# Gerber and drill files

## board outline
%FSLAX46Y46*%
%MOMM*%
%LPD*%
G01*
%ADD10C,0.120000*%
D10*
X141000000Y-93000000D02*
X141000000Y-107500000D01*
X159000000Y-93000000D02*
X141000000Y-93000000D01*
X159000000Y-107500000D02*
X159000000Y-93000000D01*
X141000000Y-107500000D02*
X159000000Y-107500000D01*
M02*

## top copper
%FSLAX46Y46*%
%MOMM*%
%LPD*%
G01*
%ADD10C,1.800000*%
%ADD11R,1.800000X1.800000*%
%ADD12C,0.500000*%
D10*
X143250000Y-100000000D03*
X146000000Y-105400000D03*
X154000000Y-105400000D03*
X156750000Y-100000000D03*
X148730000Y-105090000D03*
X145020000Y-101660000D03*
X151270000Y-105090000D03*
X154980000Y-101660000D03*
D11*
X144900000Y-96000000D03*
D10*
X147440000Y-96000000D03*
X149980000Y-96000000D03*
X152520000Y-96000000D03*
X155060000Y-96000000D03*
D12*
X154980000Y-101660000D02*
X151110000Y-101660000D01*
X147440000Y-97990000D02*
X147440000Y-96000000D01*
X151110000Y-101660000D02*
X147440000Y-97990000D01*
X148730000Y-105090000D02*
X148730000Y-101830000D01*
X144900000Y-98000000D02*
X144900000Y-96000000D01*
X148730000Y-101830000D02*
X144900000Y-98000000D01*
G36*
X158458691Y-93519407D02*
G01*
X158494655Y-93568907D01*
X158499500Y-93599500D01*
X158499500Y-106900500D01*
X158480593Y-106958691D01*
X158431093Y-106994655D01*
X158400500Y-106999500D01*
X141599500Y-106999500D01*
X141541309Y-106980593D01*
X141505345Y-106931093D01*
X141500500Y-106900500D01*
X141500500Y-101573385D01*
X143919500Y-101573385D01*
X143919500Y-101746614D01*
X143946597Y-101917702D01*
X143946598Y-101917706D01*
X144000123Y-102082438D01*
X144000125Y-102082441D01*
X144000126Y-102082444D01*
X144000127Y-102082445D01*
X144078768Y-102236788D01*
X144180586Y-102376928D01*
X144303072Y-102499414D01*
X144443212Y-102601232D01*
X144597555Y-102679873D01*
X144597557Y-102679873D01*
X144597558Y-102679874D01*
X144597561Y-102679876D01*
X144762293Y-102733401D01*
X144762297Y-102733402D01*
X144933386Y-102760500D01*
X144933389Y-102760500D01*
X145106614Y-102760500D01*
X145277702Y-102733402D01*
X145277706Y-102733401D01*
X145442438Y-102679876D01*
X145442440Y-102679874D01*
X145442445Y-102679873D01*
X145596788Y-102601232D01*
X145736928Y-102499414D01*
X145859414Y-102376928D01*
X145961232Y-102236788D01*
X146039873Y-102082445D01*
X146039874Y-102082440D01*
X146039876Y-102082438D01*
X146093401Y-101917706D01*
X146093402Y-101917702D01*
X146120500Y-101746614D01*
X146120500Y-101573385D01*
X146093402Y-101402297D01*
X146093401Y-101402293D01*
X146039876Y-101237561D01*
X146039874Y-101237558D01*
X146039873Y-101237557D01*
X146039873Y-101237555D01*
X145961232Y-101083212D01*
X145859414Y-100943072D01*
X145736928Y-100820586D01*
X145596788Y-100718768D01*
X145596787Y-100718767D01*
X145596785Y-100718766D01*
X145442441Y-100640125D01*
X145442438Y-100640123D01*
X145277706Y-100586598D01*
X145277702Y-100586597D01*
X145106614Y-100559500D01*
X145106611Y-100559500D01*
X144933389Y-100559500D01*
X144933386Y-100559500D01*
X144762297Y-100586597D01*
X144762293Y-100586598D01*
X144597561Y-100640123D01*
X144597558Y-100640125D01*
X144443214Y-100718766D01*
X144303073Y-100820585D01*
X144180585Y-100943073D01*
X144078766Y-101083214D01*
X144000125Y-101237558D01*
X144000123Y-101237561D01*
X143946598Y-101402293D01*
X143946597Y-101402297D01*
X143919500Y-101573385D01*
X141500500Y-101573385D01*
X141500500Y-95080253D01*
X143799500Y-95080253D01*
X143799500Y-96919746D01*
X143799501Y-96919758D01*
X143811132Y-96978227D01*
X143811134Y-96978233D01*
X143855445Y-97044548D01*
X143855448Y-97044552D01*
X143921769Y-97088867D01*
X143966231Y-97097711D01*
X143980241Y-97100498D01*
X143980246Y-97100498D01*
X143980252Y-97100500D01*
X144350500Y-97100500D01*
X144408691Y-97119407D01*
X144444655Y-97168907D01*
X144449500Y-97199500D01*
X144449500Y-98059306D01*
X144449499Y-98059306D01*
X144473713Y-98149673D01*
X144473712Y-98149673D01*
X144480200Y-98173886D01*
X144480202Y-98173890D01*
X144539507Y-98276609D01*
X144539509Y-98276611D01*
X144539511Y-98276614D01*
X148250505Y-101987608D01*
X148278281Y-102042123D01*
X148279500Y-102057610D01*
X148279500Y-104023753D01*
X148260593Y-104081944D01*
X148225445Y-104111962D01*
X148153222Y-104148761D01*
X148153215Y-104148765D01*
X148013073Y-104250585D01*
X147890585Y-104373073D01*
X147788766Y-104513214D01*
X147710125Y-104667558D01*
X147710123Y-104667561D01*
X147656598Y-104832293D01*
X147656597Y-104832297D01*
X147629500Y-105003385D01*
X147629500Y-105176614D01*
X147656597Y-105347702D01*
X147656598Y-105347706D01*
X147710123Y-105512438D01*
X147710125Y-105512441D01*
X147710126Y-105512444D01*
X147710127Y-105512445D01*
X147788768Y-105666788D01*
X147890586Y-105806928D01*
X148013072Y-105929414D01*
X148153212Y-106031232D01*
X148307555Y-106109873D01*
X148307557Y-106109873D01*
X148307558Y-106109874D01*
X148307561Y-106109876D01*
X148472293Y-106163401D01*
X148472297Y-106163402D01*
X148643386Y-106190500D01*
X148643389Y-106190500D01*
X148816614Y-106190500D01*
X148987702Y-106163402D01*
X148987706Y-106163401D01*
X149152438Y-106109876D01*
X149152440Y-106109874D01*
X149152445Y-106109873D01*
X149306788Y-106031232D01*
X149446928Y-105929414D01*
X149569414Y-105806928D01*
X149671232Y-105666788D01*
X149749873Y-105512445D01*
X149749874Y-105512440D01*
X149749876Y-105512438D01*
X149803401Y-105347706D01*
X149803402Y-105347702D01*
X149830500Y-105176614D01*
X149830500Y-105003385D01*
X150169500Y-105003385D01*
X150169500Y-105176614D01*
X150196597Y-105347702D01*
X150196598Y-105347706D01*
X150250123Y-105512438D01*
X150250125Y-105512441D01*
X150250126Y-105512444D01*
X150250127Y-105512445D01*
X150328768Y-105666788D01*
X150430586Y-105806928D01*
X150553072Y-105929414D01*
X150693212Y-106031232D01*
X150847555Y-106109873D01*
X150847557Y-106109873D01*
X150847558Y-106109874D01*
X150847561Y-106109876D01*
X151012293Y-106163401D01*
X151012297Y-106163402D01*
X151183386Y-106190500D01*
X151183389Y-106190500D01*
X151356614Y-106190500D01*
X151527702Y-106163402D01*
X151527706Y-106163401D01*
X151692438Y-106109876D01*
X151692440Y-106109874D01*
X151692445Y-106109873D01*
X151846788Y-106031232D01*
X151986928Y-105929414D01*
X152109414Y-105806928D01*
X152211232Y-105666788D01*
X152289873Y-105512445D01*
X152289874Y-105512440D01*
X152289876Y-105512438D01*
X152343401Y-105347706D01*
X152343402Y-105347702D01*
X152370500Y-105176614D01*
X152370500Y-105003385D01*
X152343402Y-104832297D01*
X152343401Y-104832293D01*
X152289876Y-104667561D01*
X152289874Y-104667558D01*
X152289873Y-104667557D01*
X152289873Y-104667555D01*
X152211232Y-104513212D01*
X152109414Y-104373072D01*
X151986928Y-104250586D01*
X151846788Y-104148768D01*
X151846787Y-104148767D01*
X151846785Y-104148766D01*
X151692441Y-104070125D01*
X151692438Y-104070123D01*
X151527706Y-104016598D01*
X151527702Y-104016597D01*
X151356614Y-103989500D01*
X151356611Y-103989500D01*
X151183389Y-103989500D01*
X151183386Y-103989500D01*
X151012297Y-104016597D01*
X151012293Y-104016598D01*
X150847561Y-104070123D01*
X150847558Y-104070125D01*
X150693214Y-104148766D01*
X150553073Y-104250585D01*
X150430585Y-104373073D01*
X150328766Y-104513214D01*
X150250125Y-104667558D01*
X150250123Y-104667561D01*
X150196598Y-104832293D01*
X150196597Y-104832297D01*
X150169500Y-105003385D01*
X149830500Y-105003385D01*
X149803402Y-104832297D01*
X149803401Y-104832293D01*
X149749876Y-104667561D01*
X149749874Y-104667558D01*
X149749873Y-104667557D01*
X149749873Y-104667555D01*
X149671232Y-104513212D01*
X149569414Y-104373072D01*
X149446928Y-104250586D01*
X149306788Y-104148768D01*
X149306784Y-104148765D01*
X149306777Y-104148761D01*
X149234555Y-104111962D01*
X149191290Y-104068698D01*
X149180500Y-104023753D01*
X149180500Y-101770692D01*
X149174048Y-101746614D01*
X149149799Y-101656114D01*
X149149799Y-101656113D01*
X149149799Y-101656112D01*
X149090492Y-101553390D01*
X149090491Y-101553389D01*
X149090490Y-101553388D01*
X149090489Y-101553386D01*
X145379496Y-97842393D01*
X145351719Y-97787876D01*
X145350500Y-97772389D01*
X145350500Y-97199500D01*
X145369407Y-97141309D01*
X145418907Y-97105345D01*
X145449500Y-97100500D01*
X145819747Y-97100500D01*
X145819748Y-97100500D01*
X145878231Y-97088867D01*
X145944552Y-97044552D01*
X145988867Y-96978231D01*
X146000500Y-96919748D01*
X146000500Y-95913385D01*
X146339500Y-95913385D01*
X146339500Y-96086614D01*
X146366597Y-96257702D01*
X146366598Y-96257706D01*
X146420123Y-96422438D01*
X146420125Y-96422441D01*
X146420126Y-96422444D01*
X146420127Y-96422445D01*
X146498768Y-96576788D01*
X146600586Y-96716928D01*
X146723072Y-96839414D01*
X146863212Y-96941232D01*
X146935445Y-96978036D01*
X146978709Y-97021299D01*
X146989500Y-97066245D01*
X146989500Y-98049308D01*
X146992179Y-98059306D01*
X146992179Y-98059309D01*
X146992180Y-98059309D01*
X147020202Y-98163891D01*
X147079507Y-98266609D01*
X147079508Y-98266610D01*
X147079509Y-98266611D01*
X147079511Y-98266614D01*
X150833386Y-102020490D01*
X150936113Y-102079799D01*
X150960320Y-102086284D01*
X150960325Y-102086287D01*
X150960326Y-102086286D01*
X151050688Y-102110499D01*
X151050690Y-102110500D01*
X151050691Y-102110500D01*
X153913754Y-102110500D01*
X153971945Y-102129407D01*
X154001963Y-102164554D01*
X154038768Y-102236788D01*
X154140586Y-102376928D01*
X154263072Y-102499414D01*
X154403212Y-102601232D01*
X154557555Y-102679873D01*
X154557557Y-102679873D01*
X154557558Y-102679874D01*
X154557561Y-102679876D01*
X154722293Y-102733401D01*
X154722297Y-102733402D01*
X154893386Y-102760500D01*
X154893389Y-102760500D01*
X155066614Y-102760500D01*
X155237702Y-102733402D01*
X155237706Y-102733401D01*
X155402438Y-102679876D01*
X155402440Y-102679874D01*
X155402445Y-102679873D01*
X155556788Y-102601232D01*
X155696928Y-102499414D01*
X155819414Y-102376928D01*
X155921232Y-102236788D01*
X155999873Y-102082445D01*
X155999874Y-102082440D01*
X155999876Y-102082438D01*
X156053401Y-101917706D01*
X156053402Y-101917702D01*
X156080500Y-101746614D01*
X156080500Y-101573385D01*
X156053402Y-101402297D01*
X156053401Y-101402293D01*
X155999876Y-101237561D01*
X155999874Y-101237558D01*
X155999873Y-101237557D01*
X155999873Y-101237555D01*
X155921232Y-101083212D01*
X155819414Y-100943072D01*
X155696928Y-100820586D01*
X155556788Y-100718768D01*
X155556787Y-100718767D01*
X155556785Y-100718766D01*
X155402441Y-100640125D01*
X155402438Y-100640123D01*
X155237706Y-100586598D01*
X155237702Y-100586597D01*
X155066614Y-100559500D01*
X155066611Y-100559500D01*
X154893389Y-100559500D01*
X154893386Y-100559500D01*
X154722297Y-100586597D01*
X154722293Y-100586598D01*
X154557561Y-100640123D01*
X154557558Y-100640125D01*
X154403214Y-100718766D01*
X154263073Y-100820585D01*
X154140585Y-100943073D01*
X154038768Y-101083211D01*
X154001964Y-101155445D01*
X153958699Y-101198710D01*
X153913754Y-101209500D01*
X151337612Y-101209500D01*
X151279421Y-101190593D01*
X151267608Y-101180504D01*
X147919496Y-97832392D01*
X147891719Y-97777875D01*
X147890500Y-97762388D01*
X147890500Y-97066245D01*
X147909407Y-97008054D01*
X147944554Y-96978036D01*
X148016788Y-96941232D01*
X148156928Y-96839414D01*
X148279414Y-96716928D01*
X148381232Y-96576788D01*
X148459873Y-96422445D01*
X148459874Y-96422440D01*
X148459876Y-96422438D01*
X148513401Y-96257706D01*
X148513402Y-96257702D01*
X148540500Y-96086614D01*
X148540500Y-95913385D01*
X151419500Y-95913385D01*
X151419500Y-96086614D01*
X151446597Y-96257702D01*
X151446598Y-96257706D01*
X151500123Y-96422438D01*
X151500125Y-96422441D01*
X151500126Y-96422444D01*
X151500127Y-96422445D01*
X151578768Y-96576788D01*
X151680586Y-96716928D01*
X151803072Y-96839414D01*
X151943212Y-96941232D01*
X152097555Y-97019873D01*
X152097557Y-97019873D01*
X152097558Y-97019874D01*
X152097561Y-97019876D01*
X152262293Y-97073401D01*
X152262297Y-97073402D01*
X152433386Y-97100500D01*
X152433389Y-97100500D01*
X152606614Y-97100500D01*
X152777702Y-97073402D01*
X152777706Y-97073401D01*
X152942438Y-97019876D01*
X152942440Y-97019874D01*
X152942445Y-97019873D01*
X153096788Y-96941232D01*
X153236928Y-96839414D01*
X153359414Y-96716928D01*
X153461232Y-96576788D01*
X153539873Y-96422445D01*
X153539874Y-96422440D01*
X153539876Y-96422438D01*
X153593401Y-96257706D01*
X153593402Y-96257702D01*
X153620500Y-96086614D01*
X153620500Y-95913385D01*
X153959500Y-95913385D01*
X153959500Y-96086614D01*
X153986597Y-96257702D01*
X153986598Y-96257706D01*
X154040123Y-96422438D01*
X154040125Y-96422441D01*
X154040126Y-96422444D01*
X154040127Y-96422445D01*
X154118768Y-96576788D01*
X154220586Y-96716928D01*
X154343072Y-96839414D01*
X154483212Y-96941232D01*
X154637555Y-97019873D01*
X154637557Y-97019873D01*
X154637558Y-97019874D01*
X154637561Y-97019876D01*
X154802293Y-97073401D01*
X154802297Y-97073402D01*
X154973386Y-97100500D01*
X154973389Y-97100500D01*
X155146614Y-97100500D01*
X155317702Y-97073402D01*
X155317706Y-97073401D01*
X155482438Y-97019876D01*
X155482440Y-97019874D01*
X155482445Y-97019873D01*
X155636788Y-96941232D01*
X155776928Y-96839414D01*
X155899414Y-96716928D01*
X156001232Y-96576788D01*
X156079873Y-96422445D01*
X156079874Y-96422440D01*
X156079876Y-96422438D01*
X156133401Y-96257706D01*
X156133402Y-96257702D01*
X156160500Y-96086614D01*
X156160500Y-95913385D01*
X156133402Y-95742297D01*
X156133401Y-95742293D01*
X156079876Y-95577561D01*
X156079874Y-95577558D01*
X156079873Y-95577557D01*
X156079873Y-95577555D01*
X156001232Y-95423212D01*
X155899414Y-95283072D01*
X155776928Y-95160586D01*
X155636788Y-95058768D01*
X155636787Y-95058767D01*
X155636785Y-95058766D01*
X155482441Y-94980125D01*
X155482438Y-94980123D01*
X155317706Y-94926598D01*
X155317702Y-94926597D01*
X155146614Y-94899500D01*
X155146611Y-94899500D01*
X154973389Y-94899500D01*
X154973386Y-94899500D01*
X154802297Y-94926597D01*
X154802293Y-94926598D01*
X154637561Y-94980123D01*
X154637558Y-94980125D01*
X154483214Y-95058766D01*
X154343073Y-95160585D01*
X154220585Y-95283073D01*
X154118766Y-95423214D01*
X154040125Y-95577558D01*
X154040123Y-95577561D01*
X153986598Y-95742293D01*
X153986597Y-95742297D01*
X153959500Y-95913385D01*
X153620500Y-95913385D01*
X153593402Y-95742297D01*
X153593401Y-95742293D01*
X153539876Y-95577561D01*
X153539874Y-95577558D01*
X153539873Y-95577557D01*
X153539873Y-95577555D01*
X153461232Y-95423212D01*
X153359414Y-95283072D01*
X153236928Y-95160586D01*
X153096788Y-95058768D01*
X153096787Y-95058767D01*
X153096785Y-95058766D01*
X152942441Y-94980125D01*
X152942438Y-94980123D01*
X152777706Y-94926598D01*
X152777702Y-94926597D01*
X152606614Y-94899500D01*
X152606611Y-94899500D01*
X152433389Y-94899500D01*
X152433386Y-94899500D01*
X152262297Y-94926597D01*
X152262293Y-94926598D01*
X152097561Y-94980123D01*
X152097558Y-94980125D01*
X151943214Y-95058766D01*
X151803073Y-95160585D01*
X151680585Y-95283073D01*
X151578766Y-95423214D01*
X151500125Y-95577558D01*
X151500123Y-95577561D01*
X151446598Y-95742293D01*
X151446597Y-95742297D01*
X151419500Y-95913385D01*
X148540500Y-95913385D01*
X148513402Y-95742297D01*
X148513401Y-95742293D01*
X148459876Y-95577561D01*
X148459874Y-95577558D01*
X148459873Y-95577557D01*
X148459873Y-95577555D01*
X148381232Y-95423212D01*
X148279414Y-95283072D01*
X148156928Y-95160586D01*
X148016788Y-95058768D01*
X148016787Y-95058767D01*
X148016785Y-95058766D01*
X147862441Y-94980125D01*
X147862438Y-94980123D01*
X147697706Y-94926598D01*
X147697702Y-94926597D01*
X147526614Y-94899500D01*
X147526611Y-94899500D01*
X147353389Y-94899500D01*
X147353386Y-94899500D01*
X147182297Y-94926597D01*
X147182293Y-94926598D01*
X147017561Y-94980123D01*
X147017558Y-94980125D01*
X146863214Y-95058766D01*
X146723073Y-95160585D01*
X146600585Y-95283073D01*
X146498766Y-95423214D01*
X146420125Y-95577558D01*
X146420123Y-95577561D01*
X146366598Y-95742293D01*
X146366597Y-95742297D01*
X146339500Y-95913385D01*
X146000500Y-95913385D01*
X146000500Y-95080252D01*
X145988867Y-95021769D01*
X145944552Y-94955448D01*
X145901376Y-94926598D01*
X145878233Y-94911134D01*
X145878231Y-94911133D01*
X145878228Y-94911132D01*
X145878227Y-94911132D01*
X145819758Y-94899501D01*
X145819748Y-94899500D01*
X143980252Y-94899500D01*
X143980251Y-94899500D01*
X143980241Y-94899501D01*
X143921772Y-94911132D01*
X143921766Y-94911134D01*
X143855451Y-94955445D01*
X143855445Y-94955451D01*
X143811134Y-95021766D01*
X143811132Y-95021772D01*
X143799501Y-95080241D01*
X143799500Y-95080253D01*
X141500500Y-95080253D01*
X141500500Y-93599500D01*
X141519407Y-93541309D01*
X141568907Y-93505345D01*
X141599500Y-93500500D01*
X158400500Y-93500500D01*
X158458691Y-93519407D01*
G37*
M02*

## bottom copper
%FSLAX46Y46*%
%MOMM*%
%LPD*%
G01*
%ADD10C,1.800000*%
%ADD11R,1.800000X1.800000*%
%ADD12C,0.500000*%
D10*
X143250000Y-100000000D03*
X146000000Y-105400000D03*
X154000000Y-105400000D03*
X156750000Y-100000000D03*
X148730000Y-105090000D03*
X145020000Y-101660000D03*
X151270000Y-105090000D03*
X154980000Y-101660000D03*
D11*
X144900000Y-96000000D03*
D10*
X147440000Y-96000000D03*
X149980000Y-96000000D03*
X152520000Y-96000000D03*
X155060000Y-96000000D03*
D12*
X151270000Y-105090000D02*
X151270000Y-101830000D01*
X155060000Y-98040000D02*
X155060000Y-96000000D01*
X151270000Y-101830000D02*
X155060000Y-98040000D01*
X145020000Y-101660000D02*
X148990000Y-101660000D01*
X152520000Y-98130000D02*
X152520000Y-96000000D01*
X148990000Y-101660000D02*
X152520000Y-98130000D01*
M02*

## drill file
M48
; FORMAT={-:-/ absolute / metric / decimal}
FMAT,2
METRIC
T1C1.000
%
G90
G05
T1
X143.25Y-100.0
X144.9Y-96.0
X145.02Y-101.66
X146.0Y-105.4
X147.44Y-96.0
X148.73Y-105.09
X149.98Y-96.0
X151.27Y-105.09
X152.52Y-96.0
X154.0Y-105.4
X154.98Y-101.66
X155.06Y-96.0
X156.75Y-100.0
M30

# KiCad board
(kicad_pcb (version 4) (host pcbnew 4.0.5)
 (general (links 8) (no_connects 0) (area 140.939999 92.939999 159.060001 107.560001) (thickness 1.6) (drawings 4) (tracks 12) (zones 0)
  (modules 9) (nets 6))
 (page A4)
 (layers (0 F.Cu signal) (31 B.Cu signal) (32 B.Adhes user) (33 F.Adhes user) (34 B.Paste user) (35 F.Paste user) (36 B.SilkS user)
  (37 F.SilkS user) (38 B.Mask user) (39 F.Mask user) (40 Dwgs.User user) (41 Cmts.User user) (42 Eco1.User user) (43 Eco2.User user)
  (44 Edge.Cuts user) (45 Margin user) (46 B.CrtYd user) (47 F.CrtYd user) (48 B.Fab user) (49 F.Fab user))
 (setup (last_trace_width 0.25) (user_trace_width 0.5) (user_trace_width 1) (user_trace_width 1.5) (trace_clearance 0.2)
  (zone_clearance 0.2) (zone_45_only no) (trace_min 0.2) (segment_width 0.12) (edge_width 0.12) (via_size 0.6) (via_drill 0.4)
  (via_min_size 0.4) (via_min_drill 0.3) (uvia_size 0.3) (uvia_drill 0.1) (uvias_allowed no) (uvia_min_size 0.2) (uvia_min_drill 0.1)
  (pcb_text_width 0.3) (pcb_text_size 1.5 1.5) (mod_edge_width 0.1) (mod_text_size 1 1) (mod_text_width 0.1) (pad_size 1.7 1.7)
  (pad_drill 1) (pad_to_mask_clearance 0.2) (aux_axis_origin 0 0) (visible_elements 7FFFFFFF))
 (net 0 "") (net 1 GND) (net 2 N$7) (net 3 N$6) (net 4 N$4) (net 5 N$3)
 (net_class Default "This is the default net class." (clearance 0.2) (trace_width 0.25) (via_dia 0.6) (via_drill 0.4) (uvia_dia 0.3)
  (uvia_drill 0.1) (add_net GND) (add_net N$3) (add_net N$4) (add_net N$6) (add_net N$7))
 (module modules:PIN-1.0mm (layer F.Cu) (at 143.25 100)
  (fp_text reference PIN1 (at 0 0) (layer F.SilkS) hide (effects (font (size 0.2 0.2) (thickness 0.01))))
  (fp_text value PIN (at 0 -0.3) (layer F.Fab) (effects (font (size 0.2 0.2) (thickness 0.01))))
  (pad 1 thru_hole circle (at 0 0) (size 1.8 1.8) (drill 1) (layers *.Cu *.Mask) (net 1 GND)))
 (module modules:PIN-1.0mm (layer F.Cu) (at 146 105.4)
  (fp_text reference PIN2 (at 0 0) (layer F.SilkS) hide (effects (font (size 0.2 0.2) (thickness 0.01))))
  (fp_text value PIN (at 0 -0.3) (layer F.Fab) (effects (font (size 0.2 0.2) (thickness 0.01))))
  (pad 1 thru_hole circle (at 0 0) (size 1.8 1.8) (drill 1) (layers *.Cu *.Mask) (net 1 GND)))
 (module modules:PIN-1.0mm (layer F.Cu) (at 154 105.4)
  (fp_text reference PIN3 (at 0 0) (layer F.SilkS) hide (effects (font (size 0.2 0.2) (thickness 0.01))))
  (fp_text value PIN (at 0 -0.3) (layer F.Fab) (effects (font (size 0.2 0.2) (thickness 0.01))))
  (pad 1 thru_hole circle (at 0 0) (size 1.8 1.8) (drill 1) (layers *.Cu *.Mask) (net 1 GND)))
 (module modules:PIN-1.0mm (layer F.Cu) (at 156.75 100)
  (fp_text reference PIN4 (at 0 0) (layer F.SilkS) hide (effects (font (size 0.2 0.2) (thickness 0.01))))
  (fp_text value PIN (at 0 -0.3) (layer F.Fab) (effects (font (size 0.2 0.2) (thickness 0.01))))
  (pad 1 thru_hole circle (at 0 0) (size 1.8 1.8) (drill 1) (layers *.Cu *.Mask) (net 1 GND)))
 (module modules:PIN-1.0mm (layer F.Cu) (at 148.73 105.09)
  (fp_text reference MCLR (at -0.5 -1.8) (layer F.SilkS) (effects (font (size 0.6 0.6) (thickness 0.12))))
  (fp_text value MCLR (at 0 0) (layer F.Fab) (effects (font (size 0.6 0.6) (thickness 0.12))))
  (pad 1 thru_hole circle (at 0 0) (size 1.8 1.8) (drill 1) (layers *.Cu *.Mask) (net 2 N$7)))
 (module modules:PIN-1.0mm (layer F.Cu) (at 145.02 101.66)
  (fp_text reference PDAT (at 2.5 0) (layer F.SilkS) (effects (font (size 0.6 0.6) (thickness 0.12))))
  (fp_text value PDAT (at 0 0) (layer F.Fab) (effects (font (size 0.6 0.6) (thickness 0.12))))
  (pad 1 thru_hole circle (at 0 0) (size 1.8 1.8) (drill 1) (layers *.Cu *.Mask) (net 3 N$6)))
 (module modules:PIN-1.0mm (layer F.Cu) (at 151.27 105.09)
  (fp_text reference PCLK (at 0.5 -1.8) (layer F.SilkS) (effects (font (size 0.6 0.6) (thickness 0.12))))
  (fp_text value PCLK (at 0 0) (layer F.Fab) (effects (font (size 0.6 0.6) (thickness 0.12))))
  (pad 1 thru_hole circle (at 0 0) (size 1.8 1.8) (drill 1) (layers *.Cu *.Mask) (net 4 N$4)))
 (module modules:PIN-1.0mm (layer F.Cu) (at 154.98 101.66)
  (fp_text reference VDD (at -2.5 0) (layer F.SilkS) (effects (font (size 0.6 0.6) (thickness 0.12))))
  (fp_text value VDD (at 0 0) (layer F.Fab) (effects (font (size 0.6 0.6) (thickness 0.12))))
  (pad 1 thru_hole circle (at 0 0) (size 1.8 1.8) (drill 1) (layers *.Cu *.Mask) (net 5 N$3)))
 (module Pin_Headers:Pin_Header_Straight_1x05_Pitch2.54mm (layer F.Cu) (at 144.9 96 90)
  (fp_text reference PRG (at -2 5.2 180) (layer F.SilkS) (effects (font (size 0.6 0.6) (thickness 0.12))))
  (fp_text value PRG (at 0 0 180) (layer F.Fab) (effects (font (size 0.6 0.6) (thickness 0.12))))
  (pad 1 thru_hole rect (at 0 0 90) (size 1.8 1.8) (drill 1) (layers *.Cu *.Mask) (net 2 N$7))
  (pad 2 thru_hole circle (at 0 2.54 90) (size 1.8 1.8) (drill 1) (layers *.Cu *.Mask) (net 5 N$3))
  (pad 3 thru_hole circle (at 0 5.08 90) (size 1.8 1.8) (drill 1) (layers *.Cu *.Mask) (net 1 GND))
  (pad 4 thru_hole circle (at 0 7.62 90) (size 1.8 1.8) (drill 1) (layers *.Cu *.Mask) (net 3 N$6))
  (pad 5 thru_hole circle (at 0 10.16 90) (size 1.8 1.8) (drill 1) (layers *.Cu *.Mask) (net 4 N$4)))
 (gr_line (start 141 93) (end 141 107.5) (angle 90) (layer Edge.Cuts) (width 0.12))
 (gr_line (start 159 93) (end 141 93) (angle 90) (layer Edge.Cuts) (width 0.12))
 (gr_line (start 159 107.5) (end 159 93) (angle 90) (layer Edge.Cuts) (width 0.12))
 (gr_line (start 141 107.5) (end 159 107.5) (angle 90) (layer Edge.Cuts) (width 0.12))
 (segment (start 154.98 101.66) (end 151.11 101.66) (width 0.5) (layer F.Cu) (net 5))
 (segment (start 147.44 97.99) (end 147.44 96) (width 0.5) (layer F.Cu) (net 5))
 (segment (start 151.11 101.66) (end 147.44 97.99) (width 0.5) (layer F.Cu) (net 5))
 (segment (start 151.27 105.09) (end 151.27 101.83) (width 0.5) (layer B.Cu) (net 4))
 (segment (start 155.06 98.04) (end 155.06 96) (width 0.5) (layer B.Cu) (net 4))
 (segment (start 151.27 101.83) (end 155.06 98.04) (width 0.5) (layer B.Cu) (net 4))
 (segment (start 145.02 101.66) (end 148.99 101.66) (width 0.5) (layer B.Cu) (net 3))
 (segment (start 152.52 98.13) (end 152.52 96) (width 0.5) (layer B.Cu) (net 3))
 (segment (start 148.99 101.66) (end 152.52 98.13) (width 0.5) (layer B.Cu) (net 3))
 (segment (start 148.73 105.09) (end 148.73 101.83) (width 0.5) (layer F.Cu) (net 2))
 (segment (start 144.9 98) (end 144.9 96) (width 0.5) (layer F.Cu) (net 2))
 (segment (start 148.73 101.83) (end 144.9 98) (width 0.5) (layer F.Cu) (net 2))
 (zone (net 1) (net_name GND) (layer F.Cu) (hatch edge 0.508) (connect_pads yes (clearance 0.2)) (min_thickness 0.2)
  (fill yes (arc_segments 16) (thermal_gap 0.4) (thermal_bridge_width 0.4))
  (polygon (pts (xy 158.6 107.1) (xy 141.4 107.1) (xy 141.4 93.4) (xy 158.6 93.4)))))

